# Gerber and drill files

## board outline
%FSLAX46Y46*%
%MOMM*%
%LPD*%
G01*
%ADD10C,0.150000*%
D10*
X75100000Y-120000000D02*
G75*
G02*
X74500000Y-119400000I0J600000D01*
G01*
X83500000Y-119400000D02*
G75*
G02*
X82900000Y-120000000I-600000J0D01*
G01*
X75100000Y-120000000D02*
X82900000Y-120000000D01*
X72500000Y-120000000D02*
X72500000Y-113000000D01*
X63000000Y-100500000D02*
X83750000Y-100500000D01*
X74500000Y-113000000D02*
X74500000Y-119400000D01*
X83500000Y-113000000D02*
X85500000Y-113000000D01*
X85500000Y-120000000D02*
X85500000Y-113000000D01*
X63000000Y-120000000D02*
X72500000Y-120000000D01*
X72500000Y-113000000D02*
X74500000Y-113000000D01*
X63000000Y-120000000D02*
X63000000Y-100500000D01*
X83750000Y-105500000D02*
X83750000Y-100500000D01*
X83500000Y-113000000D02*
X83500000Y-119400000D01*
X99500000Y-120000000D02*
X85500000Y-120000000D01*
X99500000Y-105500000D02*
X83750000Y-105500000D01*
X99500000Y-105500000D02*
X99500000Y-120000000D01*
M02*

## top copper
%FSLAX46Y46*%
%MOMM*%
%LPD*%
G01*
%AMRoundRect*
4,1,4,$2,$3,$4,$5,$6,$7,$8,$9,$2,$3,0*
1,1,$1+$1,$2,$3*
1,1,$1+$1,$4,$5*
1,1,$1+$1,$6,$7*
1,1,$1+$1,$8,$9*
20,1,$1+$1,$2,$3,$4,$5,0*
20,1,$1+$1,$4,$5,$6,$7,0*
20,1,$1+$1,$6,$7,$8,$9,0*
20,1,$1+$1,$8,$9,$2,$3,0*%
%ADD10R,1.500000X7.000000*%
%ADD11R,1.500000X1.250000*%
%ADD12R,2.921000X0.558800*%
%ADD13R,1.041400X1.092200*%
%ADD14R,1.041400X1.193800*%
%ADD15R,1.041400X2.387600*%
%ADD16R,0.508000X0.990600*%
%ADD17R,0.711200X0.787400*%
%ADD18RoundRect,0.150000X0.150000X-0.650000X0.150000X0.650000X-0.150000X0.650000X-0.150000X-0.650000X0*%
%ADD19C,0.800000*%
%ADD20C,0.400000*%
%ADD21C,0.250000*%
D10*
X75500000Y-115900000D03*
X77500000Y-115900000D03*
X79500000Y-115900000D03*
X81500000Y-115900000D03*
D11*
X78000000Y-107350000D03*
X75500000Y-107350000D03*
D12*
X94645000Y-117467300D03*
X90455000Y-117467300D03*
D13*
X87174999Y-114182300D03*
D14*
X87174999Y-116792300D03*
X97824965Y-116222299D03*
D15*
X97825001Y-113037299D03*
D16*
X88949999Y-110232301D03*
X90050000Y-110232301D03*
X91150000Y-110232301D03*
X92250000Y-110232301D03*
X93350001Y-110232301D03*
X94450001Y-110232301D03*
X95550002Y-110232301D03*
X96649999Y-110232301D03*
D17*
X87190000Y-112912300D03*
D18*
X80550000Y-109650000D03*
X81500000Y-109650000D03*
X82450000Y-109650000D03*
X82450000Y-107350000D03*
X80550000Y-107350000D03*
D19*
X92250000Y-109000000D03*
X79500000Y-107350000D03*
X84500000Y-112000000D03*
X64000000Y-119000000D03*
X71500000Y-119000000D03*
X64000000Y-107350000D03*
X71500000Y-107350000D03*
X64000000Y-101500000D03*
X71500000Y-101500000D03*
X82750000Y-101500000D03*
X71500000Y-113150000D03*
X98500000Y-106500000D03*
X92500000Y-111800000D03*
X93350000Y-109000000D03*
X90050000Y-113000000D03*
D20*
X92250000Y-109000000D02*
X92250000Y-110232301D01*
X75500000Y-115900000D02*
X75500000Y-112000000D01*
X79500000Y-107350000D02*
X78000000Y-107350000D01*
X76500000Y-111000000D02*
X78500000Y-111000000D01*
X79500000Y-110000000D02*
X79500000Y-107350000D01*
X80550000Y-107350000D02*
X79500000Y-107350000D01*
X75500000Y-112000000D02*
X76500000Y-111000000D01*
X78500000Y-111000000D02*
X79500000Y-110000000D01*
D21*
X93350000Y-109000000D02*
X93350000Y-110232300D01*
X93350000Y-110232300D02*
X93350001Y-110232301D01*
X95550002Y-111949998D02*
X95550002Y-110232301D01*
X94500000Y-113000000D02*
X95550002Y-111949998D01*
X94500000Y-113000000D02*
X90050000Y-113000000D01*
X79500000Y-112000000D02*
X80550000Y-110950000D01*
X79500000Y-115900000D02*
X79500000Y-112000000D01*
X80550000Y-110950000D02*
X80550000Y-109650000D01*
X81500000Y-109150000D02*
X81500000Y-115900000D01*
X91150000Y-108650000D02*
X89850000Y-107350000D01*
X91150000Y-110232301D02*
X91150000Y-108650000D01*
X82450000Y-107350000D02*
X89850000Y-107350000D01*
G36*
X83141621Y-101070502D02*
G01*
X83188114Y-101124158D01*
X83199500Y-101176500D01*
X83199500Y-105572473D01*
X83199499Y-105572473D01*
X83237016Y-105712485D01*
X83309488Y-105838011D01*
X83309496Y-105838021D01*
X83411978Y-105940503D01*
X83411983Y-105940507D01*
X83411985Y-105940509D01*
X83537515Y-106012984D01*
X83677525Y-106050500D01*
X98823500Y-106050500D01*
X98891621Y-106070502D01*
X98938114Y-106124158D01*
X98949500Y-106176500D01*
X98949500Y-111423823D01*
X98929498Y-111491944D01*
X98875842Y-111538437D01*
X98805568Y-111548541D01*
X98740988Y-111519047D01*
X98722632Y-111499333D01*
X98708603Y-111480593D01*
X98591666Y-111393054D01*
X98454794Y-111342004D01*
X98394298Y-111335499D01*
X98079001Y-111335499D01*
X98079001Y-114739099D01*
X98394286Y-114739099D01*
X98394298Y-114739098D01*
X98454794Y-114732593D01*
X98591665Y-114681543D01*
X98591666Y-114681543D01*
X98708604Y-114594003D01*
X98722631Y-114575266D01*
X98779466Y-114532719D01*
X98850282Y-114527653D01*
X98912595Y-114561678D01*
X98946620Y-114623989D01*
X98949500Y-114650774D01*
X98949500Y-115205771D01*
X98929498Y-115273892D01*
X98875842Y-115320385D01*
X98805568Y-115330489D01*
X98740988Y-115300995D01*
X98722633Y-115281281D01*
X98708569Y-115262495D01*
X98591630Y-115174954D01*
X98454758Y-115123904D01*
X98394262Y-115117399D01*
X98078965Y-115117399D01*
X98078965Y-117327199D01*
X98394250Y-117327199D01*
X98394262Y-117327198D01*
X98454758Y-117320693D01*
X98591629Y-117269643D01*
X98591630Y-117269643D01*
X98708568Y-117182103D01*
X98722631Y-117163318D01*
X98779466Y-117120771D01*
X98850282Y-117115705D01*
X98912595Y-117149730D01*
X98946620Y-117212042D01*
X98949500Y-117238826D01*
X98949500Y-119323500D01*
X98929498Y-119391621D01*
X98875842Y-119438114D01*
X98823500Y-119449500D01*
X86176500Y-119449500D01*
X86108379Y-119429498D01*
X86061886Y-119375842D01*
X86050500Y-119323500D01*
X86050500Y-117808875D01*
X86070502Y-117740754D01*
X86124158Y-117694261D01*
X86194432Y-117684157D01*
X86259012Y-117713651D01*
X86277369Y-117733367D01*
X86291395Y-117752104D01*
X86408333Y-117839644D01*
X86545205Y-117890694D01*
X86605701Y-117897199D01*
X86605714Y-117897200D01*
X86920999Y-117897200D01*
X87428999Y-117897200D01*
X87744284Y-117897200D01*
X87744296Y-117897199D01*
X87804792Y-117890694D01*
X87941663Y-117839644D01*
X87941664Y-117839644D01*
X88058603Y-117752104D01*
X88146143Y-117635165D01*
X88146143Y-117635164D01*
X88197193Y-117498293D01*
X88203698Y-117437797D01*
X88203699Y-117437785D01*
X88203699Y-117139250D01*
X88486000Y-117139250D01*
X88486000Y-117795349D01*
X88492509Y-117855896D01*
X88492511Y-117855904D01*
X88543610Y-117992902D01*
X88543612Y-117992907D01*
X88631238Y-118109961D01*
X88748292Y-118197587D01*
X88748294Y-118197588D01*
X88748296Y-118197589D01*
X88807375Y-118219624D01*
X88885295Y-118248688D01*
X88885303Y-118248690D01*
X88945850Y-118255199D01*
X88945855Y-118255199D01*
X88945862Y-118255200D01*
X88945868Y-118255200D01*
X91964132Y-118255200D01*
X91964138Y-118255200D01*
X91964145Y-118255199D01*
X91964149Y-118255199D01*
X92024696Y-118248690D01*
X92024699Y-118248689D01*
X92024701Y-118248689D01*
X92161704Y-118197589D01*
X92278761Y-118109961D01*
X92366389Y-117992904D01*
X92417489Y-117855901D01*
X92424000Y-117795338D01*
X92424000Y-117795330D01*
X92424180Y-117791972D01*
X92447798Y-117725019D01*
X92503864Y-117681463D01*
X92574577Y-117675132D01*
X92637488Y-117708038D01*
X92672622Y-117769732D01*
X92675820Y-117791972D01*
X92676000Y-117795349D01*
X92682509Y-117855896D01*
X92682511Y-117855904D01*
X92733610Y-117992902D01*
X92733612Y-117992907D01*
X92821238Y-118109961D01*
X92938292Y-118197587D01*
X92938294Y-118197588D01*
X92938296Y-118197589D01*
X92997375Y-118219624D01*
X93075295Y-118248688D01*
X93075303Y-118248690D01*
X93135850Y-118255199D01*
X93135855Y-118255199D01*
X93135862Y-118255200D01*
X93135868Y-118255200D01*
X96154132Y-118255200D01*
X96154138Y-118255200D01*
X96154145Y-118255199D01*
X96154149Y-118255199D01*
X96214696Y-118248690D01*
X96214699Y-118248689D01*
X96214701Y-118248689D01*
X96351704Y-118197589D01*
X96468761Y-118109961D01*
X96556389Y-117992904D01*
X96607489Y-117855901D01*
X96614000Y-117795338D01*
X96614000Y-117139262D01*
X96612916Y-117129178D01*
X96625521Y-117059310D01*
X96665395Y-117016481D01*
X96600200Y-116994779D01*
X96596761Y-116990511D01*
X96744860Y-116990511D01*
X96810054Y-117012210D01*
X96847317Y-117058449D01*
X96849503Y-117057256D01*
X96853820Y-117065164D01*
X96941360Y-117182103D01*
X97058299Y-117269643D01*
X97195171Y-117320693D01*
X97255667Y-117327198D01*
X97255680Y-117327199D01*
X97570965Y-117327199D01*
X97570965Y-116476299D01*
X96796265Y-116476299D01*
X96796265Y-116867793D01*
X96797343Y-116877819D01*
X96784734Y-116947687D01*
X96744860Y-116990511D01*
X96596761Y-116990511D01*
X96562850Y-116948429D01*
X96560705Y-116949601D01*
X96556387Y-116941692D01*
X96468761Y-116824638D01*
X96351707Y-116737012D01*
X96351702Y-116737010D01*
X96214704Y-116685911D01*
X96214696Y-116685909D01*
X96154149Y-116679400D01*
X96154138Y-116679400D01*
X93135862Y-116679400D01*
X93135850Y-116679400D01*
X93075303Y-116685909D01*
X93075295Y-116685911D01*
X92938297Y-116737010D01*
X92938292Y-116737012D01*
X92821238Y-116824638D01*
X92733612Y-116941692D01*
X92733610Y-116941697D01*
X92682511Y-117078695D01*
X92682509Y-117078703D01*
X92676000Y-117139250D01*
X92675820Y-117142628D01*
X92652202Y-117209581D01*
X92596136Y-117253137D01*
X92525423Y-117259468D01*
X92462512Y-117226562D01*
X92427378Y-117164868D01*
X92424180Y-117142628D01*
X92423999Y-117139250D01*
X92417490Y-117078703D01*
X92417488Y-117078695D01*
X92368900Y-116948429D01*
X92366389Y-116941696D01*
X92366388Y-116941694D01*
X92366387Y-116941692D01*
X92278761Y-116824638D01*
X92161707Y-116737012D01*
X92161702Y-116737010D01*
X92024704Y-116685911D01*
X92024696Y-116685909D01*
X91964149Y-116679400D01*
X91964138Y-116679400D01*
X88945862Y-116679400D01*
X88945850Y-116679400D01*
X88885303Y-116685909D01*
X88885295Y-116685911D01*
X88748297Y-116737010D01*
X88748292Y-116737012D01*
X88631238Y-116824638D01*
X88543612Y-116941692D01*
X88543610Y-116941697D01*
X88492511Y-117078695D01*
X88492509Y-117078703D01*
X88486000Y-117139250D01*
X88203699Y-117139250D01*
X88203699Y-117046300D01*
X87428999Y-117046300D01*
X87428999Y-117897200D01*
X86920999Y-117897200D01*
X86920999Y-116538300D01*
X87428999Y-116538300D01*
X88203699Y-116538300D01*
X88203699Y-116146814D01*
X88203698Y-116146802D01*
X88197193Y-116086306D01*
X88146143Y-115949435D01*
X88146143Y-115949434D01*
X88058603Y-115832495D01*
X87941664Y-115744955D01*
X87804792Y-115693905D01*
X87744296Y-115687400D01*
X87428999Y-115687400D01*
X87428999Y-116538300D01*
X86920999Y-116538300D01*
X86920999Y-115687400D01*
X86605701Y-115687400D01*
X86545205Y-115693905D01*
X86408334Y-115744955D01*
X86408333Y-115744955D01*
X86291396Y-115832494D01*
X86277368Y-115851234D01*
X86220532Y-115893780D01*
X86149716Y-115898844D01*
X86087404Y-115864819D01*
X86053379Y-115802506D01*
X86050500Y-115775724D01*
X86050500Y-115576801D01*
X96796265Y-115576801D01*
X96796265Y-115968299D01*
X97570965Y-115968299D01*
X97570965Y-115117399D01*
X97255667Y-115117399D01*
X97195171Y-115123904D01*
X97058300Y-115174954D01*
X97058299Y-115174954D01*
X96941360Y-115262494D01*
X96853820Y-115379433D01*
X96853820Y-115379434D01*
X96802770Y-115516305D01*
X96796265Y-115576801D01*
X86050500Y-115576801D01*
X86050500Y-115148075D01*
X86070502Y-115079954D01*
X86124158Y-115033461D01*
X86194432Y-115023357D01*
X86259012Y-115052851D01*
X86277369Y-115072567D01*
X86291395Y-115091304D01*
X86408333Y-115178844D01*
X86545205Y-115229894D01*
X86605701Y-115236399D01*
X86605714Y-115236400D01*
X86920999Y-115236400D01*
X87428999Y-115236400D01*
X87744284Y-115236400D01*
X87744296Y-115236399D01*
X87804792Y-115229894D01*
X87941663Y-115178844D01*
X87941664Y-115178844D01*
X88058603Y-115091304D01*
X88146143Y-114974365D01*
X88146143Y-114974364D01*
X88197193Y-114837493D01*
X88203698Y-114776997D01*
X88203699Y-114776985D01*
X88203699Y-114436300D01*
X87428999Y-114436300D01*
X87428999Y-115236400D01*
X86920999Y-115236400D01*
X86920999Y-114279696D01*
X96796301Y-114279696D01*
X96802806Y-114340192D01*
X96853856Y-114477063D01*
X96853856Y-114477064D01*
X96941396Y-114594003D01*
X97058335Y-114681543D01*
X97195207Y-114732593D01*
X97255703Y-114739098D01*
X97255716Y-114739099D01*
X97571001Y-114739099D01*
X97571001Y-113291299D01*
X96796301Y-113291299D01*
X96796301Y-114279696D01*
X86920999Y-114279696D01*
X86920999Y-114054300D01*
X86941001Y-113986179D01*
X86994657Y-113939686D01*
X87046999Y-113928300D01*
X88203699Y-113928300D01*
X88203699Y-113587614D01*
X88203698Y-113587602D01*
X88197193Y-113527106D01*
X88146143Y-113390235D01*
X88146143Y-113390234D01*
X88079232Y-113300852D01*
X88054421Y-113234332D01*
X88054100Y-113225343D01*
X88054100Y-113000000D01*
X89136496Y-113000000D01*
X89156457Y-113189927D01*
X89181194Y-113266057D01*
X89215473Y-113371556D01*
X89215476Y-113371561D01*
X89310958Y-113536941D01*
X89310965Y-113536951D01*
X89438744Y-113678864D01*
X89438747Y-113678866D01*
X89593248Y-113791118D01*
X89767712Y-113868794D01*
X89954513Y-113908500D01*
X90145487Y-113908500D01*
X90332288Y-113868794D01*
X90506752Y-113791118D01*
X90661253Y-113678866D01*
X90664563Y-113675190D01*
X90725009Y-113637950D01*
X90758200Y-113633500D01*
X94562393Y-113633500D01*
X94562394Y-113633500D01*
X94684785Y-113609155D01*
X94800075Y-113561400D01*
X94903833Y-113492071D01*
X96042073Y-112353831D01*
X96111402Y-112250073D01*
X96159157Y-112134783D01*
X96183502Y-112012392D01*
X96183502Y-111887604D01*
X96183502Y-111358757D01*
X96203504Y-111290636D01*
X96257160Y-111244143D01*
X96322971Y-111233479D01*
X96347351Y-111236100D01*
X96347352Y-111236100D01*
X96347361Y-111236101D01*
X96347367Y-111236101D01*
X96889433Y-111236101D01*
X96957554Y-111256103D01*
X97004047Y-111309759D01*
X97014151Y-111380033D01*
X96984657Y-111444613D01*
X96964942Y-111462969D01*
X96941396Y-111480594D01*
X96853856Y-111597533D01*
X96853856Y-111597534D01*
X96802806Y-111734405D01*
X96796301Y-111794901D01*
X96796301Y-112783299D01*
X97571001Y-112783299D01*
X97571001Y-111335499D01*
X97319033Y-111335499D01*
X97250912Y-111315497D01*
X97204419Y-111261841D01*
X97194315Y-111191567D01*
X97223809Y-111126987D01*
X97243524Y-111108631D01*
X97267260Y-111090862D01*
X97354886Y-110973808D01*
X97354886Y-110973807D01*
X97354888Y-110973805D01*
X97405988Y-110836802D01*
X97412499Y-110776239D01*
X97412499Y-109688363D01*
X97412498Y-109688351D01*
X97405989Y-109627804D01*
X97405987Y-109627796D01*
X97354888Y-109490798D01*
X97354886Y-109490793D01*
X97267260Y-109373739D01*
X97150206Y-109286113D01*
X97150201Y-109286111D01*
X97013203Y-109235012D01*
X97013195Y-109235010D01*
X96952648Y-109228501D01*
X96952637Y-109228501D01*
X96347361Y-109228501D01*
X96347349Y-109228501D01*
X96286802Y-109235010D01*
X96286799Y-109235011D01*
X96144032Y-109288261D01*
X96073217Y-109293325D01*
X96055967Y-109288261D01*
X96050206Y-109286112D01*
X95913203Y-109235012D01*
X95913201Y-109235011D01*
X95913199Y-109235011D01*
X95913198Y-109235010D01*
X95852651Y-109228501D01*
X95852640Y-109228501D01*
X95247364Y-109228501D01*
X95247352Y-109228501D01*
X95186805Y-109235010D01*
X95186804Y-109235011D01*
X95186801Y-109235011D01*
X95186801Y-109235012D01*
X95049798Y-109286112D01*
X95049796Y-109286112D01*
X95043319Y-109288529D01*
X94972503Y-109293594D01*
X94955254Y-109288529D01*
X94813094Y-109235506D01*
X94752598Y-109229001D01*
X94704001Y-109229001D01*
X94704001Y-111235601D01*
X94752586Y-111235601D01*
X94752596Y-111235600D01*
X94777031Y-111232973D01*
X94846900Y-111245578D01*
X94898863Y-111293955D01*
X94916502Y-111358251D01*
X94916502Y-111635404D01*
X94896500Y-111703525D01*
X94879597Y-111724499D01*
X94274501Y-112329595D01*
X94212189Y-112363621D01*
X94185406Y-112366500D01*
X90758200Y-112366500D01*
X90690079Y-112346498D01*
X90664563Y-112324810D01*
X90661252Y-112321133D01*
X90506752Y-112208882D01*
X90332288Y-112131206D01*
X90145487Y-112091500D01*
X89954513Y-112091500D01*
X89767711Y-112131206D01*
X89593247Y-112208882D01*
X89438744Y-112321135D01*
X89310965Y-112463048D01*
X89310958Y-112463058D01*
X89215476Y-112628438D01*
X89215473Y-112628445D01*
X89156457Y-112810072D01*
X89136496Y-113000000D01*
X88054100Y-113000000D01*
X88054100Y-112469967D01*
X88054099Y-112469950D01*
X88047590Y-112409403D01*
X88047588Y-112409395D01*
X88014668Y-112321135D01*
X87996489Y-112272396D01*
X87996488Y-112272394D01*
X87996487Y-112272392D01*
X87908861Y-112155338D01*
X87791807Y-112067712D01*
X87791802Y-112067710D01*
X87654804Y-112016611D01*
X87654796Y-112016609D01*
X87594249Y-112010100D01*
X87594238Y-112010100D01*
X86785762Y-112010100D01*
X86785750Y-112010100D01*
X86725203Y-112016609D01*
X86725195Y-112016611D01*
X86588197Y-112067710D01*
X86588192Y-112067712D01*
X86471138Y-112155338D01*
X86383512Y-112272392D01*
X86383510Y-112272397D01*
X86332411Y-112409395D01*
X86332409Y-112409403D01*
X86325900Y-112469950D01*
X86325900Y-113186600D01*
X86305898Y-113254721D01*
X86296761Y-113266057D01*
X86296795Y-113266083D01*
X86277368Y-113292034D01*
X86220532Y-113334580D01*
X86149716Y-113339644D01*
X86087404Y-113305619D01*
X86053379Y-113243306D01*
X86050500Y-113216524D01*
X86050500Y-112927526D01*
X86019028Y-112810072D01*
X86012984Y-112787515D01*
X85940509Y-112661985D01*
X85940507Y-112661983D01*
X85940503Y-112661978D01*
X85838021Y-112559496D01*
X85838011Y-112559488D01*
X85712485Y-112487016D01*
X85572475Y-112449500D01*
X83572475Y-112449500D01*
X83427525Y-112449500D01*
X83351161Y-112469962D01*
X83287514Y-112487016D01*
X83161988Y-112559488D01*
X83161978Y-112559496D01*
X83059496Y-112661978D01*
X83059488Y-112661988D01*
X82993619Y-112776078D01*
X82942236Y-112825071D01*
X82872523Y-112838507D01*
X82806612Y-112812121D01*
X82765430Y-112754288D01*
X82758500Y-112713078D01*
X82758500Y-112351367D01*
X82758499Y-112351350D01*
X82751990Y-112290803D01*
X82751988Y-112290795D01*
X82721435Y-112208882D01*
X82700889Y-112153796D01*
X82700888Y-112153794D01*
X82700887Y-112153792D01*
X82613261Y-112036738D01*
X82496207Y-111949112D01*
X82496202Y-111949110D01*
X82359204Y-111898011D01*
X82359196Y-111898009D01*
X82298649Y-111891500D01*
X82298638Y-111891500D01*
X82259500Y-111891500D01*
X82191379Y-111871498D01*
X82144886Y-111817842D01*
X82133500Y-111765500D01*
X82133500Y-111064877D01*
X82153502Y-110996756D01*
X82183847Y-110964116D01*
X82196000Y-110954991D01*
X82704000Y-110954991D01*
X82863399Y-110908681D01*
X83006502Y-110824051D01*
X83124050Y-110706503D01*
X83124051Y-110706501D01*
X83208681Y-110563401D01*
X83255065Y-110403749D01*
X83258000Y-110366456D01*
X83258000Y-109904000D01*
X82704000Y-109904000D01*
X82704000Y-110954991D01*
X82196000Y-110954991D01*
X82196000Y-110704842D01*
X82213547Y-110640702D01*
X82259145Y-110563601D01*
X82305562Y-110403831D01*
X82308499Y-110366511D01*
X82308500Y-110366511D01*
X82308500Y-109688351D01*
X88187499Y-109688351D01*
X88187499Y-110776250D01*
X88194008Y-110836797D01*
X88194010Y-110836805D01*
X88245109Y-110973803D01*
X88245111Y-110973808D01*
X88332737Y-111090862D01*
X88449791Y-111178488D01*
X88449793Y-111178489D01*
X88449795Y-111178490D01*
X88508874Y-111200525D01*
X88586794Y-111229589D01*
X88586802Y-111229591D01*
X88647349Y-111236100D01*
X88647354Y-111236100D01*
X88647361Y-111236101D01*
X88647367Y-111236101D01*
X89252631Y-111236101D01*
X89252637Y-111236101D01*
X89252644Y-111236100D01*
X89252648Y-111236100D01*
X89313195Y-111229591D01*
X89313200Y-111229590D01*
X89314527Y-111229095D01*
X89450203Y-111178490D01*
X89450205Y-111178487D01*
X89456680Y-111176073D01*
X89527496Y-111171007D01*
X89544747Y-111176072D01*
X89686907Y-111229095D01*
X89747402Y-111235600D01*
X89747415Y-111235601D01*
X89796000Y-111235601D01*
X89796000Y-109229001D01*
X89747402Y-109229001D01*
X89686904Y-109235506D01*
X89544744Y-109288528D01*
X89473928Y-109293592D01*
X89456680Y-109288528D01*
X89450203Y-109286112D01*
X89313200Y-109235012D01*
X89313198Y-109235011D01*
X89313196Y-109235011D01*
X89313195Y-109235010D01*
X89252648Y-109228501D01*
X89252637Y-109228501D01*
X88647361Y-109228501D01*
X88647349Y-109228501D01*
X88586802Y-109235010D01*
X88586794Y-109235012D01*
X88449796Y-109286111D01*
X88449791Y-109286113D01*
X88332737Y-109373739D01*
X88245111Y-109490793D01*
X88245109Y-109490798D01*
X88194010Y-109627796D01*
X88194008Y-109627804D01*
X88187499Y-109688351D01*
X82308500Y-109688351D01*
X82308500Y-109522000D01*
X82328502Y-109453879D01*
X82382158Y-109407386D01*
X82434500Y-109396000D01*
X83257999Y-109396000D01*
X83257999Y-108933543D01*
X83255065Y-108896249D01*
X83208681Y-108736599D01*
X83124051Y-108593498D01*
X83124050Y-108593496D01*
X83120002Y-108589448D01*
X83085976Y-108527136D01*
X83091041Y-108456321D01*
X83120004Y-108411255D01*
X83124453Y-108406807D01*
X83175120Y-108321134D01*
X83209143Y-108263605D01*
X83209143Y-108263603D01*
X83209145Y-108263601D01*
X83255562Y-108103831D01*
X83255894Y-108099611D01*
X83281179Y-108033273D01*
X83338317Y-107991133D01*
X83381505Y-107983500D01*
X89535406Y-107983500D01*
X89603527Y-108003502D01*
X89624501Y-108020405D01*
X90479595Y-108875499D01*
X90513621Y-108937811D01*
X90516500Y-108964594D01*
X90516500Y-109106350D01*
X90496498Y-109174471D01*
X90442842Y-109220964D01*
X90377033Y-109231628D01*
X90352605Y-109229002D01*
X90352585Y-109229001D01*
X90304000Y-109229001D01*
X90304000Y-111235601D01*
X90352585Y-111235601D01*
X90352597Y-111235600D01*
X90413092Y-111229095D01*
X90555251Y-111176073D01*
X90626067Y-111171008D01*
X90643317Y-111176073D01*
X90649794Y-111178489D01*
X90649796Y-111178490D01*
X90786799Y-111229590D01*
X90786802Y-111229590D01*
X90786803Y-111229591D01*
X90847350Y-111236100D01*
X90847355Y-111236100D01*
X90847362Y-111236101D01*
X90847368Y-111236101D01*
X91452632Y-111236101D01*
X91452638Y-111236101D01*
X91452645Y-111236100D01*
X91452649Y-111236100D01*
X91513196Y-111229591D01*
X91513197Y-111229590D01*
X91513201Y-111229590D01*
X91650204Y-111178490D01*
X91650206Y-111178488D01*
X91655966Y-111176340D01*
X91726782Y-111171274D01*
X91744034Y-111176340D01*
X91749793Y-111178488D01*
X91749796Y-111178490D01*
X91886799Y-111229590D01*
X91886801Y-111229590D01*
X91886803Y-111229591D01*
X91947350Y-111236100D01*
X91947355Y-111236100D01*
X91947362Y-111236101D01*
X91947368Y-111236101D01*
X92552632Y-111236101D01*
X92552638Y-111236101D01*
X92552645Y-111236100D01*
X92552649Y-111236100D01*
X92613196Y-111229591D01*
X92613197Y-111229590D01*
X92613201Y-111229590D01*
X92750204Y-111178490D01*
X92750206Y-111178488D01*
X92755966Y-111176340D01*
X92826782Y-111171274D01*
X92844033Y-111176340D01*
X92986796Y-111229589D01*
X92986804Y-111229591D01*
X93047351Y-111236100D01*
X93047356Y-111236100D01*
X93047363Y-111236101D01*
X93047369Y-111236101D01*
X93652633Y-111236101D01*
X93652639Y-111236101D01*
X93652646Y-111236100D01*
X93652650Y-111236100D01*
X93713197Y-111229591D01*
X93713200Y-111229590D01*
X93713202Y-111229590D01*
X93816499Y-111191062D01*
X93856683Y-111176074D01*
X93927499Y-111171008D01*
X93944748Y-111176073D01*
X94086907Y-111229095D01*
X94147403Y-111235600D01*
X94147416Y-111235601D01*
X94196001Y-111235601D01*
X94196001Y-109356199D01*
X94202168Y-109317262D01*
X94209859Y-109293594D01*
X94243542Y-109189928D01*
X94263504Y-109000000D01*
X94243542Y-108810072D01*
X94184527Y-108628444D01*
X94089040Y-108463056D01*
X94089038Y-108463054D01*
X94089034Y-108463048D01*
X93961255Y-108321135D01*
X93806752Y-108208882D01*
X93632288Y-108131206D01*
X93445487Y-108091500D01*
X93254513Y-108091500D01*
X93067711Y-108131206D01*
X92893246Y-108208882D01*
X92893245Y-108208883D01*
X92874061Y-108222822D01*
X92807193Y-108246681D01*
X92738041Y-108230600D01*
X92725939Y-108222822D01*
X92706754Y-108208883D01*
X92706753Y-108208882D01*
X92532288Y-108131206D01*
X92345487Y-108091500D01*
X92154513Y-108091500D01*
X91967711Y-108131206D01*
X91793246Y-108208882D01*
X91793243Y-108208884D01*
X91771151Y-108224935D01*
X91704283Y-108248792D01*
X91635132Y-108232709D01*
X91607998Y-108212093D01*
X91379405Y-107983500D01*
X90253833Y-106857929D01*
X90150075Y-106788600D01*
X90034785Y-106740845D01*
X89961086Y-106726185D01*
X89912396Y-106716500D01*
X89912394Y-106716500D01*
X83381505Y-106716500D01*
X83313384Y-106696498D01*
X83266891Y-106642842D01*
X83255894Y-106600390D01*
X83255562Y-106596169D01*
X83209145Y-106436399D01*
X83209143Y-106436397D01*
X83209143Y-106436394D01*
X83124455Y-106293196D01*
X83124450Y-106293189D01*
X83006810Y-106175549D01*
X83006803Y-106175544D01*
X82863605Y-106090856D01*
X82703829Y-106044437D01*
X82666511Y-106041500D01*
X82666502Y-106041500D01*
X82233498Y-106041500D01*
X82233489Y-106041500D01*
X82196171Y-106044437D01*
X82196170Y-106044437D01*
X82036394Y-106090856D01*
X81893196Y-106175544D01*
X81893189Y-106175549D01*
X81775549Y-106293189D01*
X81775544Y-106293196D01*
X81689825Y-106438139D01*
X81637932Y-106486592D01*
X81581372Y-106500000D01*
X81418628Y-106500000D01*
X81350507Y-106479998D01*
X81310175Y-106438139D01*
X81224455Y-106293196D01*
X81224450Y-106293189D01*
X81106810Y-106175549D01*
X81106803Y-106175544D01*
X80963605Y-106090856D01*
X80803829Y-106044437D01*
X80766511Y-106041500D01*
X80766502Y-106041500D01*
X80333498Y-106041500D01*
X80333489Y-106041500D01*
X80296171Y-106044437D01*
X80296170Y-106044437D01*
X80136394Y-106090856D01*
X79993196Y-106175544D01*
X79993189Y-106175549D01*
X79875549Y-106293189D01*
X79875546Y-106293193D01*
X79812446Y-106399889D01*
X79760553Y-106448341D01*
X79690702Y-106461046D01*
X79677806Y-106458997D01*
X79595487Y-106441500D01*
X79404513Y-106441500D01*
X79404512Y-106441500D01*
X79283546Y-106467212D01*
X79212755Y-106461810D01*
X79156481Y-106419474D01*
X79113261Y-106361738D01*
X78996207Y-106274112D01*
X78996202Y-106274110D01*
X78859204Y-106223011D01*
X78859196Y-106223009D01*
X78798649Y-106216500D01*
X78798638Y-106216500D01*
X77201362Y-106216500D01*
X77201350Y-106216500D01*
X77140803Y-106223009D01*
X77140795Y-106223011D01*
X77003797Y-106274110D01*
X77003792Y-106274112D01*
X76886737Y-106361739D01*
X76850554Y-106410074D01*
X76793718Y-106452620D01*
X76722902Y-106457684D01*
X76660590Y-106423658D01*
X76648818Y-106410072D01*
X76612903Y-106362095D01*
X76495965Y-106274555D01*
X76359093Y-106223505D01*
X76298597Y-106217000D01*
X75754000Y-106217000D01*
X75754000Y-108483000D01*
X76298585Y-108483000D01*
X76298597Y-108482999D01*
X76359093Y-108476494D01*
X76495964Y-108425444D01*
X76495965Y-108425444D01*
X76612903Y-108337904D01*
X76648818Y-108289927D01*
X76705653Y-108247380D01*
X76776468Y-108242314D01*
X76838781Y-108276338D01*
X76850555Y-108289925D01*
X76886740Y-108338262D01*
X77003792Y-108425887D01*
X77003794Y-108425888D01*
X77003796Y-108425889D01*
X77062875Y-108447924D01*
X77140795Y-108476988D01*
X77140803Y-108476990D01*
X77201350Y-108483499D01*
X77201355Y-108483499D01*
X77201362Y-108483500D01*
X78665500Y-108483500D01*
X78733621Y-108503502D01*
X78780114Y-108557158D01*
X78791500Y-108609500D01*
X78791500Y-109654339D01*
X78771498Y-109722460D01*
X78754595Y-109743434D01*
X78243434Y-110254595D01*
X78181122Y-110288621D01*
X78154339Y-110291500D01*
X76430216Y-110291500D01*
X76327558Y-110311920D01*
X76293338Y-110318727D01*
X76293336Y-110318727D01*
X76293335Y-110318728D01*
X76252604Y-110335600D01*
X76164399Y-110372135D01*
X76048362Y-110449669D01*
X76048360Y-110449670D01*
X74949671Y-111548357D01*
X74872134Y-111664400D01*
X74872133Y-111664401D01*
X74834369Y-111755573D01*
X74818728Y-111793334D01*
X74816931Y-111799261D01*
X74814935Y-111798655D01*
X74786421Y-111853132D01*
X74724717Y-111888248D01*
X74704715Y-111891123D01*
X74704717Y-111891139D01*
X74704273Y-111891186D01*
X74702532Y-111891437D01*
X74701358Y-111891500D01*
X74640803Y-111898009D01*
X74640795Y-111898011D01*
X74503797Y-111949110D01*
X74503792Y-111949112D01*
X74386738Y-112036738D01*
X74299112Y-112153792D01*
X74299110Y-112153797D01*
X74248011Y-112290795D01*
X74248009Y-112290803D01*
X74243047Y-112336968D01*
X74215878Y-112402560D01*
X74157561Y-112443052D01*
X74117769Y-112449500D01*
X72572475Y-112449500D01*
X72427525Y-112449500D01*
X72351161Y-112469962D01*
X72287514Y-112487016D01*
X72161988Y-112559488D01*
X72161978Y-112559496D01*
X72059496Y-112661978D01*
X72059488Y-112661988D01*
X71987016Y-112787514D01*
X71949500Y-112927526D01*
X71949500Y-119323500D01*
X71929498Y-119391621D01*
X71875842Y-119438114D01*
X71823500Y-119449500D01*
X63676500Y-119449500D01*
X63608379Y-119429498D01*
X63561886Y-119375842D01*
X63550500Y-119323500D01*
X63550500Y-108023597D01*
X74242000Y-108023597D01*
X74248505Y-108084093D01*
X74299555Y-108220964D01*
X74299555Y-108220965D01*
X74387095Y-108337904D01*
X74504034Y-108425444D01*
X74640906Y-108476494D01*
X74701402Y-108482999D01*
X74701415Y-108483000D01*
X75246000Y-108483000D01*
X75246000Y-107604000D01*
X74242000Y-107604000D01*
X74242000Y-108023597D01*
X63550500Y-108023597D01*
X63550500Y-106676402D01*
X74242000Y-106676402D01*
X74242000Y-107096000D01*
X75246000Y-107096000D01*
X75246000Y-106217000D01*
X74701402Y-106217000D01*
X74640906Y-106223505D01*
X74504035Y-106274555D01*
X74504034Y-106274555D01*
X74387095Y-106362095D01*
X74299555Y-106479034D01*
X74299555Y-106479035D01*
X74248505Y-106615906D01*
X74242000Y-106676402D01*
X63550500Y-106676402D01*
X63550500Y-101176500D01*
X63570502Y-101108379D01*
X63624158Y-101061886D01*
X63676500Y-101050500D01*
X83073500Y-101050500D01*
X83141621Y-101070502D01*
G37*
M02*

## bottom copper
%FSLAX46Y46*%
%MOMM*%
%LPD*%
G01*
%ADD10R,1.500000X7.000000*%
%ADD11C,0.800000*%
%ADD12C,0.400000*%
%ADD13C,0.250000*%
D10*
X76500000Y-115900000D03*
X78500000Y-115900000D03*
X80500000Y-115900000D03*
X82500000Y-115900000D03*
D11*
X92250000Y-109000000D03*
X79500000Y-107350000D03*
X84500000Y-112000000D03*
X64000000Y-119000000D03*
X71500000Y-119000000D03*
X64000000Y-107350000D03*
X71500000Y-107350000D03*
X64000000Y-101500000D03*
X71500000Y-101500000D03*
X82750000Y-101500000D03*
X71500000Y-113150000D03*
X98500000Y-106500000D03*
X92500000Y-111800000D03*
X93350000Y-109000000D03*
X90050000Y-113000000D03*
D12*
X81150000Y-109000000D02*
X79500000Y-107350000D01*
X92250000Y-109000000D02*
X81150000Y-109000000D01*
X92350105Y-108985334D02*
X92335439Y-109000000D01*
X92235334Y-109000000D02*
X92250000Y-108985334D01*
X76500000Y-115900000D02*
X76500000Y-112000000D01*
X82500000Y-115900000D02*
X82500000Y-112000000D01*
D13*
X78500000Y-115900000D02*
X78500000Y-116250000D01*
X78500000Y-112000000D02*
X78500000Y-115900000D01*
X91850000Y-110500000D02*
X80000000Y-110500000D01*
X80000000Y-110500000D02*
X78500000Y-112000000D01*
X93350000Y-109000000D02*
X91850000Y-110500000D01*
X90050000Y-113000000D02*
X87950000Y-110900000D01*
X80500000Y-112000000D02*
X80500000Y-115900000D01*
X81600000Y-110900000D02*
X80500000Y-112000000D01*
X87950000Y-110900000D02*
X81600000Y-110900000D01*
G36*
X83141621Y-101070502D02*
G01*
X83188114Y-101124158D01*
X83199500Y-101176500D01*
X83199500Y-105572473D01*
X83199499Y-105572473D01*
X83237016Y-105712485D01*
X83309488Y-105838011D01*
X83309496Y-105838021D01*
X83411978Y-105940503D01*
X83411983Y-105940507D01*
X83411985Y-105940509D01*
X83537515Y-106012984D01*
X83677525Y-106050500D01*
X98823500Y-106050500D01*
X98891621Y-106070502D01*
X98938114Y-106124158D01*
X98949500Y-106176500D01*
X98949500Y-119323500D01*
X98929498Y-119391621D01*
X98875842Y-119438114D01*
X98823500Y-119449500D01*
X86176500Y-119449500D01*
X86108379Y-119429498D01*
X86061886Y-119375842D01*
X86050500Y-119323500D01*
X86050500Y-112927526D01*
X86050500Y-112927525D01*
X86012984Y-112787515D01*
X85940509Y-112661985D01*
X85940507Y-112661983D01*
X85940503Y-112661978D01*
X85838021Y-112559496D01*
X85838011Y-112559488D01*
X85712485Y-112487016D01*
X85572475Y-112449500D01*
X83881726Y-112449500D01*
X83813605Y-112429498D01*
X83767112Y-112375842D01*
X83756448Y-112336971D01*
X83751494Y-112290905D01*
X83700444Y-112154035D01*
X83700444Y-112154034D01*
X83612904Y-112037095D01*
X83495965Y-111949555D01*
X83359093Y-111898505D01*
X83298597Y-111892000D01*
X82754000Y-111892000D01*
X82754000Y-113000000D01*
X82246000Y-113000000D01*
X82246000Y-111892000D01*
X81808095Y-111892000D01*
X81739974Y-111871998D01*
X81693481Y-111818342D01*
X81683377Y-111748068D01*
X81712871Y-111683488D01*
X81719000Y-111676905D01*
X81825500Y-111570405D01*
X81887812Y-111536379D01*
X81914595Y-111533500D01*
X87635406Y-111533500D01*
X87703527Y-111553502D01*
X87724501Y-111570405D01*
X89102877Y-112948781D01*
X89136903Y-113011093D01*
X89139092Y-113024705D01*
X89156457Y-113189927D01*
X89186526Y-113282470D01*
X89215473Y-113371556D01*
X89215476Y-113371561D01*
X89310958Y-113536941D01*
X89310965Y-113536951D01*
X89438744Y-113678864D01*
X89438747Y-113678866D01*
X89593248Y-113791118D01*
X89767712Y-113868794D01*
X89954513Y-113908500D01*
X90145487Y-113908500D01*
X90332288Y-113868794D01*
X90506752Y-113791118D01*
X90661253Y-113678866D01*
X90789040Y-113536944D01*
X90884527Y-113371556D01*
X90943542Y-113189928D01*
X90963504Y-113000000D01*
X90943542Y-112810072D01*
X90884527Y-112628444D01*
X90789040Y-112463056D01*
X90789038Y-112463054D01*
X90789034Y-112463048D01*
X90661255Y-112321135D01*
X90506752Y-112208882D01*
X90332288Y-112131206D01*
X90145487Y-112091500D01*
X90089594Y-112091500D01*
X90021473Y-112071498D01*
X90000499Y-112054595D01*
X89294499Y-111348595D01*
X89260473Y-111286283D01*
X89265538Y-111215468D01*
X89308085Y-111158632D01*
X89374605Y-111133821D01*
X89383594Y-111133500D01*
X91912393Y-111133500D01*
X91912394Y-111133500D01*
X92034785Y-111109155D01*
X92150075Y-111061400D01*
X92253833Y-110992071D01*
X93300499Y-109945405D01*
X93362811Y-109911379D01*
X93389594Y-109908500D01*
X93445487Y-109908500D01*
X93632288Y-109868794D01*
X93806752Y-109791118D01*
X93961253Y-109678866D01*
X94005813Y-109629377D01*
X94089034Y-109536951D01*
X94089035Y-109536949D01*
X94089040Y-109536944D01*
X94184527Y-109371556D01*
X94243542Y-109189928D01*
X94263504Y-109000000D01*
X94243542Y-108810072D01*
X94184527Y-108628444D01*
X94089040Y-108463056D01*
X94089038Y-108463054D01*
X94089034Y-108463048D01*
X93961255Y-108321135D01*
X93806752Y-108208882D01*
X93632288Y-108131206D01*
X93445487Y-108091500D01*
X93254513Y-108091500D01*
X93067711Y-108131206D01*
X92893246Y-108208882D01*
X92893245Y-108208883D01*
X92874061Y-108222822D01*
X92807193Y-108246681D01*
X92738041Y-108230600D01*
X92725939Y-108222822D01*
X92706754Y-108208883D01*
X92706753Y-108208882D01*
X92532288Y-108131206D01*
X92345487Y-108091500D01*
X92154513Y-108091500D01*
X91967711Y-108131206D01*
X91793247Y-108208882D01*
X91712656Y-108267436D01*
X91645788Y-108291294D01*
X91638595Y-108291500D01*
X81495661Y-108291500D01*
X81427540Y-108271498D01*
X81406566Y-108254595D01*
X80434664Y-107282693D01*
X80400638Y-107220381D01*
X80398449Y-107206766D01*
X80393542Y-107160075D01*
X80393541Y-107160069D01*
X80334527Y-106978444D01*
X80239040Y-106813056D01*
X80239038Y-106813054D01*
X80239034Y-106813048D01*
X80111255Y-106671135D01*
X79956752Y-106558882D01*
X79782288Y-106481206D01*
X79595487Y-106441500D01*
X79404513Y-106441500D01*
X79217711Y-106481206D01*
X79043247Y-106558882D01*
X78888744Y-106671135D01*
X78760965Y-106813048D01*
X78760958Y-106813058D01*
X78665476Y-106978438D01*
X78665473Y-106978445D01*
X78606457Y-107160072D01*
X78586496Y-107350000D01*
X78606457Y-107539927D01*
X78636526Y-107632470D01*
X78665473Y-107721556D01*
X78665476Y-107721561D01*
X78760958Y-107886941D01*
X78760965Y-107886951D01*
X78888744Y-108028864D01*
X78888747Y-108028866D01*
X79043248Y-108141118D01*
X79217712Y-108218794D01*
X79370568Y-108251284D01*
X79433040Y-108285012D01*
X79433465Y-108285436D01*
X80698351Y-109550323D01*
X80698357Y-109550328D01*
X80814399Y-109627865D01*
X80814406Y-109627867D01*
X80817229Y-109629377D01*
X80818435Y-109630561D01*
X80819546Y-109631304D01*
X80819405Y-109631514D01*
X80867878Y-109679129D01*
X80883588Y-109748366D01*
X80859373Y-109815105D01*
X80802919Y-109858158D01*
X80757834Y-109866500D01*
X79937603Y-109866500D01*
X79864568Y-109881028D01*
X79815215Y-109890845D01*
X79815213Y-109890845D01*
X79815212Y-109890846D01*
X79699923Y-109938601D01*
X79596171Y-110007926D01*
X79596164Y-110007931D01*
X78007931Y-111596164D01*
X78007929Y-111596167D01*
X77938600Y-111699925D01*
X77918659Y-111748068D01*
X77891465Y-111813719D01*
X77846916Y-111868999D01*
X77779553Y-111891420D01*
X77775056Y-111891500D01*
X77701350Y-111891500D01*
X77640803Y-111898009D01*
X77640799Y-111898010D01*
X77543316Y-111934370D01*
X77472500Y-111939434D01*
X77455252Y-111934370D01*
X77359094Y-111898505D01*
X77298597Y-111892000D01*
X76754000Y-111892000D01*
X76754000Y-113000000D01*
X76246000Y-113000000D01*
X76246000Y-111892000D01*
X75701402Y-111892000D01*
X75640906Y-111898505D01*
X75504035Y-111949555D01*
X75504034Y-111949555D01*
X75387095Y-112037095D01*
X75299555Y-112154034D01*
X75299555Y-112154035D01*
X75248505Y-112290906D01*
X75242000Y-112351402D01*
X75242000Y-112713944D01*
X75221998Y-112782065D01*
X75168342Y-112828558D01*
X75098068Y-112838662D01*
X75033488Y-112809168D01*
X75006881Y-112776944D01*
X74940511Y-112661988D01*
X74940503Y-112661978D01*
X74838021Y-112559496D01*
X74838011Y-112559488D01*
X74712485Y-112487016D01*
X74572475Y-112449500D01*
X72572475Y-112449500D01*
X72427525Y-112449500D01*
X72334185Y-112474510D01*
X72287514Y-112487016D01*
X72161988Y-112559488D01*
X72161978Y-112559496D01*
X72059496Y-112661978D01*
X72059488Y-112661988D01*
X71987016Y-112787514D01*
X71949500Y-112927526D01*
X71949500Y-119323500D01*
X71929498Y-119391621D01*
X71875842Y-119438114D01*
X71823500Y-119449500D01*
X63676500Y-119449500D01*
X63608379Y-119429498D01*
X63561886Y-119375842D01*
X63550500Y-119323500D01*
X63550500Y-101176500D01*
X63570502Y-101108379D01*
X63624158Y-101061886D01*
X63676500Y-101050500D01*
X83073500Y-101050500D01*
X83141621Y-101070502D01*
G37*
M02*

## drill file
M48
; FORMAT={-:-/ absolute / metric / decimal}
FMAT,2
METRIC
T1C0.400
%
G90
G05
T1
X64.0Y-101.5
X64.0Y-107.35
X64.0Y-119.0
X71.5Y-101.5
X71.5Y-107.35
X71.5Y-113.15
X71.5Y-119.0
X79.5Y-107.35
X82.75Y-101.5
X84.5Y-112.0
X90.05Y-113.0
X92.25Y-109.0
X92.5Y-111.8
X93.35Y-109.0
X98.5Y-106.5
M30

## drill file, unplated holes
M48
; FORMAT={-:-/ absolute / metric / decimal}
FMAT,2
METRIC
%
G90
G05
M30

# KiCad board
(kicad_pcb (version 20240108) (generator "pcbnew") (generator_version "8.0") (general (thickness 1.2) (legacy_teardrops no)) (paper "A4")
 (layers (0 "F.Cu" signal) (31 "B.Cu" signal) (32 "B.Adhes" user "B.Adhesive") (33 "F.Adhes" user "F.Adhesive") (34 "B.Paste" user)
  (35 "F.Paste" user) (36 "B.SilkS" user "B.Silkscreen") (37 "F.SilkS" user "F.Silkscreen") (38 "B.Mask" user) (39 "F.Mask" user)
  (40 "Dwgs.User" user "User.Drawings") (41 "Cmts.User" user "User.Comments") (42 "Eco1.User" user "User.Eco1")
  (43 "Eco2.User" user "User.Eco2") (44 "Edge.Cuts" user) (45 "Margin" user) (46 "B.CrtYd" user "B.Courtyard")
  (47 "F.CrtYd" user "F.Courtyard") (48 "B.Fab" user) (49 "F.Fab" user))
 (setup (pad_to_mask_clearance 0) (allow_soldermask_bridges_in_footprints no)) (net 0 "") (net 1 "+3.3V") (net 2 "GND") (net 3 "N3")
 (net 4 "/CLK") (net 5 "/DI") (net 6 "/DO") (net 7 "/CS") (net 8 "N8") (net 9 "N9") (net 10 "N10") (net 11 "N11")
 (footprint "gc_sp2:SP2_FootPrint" (layer "F.Cu") (at 75.5 115.9)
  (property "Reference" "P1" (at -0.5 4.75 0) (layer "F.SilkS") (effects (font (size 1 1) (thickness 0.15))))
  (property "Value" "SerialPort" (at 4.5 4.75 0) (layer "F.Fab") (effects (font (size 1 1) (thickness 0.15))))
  (pad "1" smd rect (at 0 0) (size 1.5 7) (layers "F.Cu" "F.Mask") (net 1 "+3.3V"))
  (pad "2" smd rect (at 1 0) (size 1.5 7) (layers "B.Cu" "B.Mask") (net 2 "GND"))
  (pad "3" smd rect (at 2 0) (size 1.5 7) (layers "F.Cu" "F.Mask") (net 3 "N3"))
  (pad "4" smd rect (at 3 0) (size 1.5 7) (layers "B.Cu" "B.Mask") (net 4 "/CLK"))
  (pad "5" smd rect (at 4 0) (size 1.5 7) (layers "F.Cu" "F.Mask") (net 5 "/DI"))
  (pad "6" smd rect (at 5 0) (size 1.5 7) (layers "B.Cu" "B.Mask") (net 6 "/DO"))
  (pad "7" smd rect (at 6 0) (size 1.5 7) (layers "F.Cu" "F.Mask") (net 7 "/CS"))
  (pad "8" smd rect (at 7 0) (size 1.5 7) (layers "B.Cu" "B.Mask") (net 2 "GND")))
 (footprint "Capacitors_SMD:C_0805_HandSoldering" (layer "F.Cu") (at 76.75 107.35 180)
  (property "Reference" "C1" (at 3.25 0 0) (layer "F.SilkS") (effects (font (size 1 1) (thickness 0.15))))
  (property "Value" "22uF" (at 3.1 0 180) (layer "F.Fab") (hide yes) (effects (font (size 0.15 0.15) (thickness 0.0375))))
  (pad "1" smd rect (at -1.25 0 180) (size 1.5 1.25) (layers "F.Cu" "F.Paste" "F.Mask") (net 1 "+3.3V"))
  (pad "2" smd rect (at 1.25 0 180) (size 1.5 1.25) (layers "F.Cu" "F.Paste" "F.Mask") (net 2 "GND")))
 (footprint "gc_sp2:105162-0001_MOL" (layer "F.Cu") (at 92.5 113.75 180)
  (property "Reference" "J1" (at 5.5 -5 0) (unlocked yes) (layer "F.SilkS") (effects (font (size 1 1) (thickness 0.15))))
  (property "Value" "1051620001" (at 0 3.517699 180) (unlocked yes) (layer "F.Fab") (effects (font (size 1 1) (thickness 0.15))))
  (pad "14" smd rect (at -2.145 -3.7173 180) (size 2.921 0.5588) (layers "F.Cu" "F.Paste" "F.Mask"))
  (pad "15" smd rect (at 2.045 -3.7173 180) (size 2.921 0.5588) (layers "F.Cu" "F.Paste" "F.Mask"))
  (pad "G1" smd rect (at 5.325001 -0.4323 180) (size 1.0414 1.0922) (layers "F.Cu" "F.Paste" "F.Mask") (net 2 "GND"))
  (pad "G2" smd rect (at 5.325001 -3.0423 180) (size 1.0414 1.1938) (layers "F.Cu" "F.Paste" "F.Mask") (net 2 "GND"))
  (pad "G3" smd rect (at -5.324965 -2.472299 180) (size 1.0414 1.1938) (layers "F.Cu" "F.Paste" "F.Mask") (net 2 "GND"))
  (pad "G4" smd rect (at -5.325001 0.712701 180) (size 1.0414 2.3876) (layers "F.Cu" "F.Paste" "F.Mask") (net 2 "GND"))
  (pad "P1" smd rect (at 3.550001 3.517699 180) (size 0.508 0.9906) (layers "F.Cu" "F.Paste" "F.Mask") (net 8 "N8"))
  (pad "P2" smd rect (at 2.45 3.517699 180) (size 0.508 0.9906) (layers "F.Cu" "F.Paste" "F.Mask") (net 2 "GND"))
  (pad "P3" smd rect (at 1.35 3.517699 180) (size 0.508 0.9906) (layers "F.Cu" "F.Paste" "F.Mask") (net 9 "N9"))
  (pad "P4" smd rect (at 0.25 3.517699 180) (size 0.508 0.9906) (layers "F.Cu" "F.Paste" "F.Mask") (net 1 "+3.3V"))
  (pad "P5" smd rect (at -0.850001 3.517699 180) (size 0.508 0.9906) (layers "F.Cu" "F.Paste" "F.Mask") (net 4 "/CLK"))
  (pad "P6" smd rect (at -1.950001 3.517699 180) (size 0.508 0.9906) (layers "F.Cu" "F.Paste" "F.Mask") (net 2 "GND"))
  (pad "P7" smd rect (at -3.050002 3.517699 180) (size 0.508 0.9906) (layers "F.Cu" "F.Paste" "F.Mask") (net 6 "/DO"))
  (pad "P8" smd rect (at -4.149999 3.517699 180) (size 0.508 0.9906) (layers "F.Cu" "F.Paste" "F.Mask") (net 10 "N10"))
  (pad "P9" smd rect (at 5.31 0.8377 180) (size 0.7112 0.7874) (layers "F.Cu" "F.Paste" "F.Mask") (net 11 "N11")))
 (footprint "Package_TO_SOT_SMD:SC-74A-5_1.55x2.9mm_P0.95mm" (layer "F.Cu") (at 81.5 108.5 90)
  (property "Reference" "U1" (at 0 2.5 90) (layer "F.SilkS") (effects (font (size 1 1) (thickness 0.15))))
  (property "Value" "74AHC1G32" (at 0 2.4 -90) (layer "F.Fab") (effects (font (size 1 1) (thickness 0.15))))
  (pad "1" smd roundrect (at -1.15 -0.95 90) (size 1.6 0.6) (layers "F.Cu" "F.Paste" "F.Mask") (roundrect_rratio 0.25) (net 5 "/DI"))
  (pad "2" smd roundrect (at -1.15 0 90) (size 1.6 0.6) (layers "F.Cu" "F.Paste" "F.Mask") (roundrect_rratio 0.25) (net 7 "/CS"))
  (pad "3" smd roundrect (at -1.15 0.95 90) (size 1.6 0.6) (layers "F.Cu" "F.Paste" "F.Mask") (roundrect_rratio 0.25) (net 2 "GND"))
  (pad "4" smd roundrect (at 1.15 0.95 90) (size 1.6 0.6) (layers "F.Cu" "F.Paste" "F.Mask") (roundrect_rratio 0.25) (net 9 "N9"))
  (pad "5" smd roundrect (at 1.15 -0.95 90) (size 1.6 0.6) (layers "F.Cu" "F.Paste" "F.Mask") (roundrect_rratio 0.25) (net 1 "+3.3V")))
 (gr_arc (start 75.1 120) (mid 74.675736 119.824264) (end 74.5 119.4) (stroke (width 0.15) (type solid)) (layer "Edge.Cuts"))
 (gr_arc (start 83.5 119.4) (mid 83.324264 119.824264) (end 82.9 120) (stroke (width 0.15) (type solid)) (layer "Edge.Cuts"))
 (gr_line (start 75.1 120) (end 82.9 120) (stroke (width 0.15) (type solid)) (layer "Edge.Cuts"))
 (gr_line (start 72.5 120) (end 72.5 113) (stroke (width 0.15) (type solid)) (layer "Edge.Cuts"))
 (gr_line (start 63 100.5) (end 83.75 100.5) (stroke (width 0.15) (type solid)) (layer "Edge.Cuts"))
 (gr_line (start 74.5 113) (end 74.5 119.4) (stroke (width 0.15) (type solid)) (layer "Edge.Cuts"))
 (gr_line (start 83.5 113) (end 85.5 113) (stroke (width 0.15) (type solid)) (layer "Edge.Cuts"))
 (gr_line (start 85.5 120) (end 85.5 113) (stroke (width 0.15) (type solid)) (layer "Edge.Cuts"))
 (gr_line (start 63 120) (end 72.5 120) (stroke (width 0.15) (type solid)) (layer "Edge.Cuts"))
 (gr_line (start 72.5 113) (end 74.5 113) (stroke (width 0.15) (type solid)) (layer "Edge.Cuts"))
 (gr_line (start 63 120) (end 63 100.5) (stroke (width 0.15) (type solid)) (layer "Edge.Cuts"))
 (gr_line (start 83.75 105.5) (end 83.75 100.5) (stroke (width 0.15) (type solid)) (layer "Edge.Cuts"))
 (gr_line (start 83.5 113) (end 83.5 119.4) (stroke (width 0.15) (type solid)) (layer "Edge.Cuts"))
 (gr_line (start 99.5 120) (end 85.5 120) (stroke (width 0.15) (type solid)) (layer "Edge.Cuts"))
 (gr_line (start 99.5 105.5) (end 83.75 105.5) (stroke (width 0.15) (type solid)) (layer "Edge.Cuts"))
 (gr_line (start 99.5 105.5) (end 99.5 120) (stroke (width 0.15) (type solid)) (layer "Edge.Cuts"))
 (segment (start 92.25 109) (end 92.25 110.232301) (width 0.4) (layer "F.Cu") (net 1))
 (segment (start 75.5 115.9) (end 75.5 112) (width 0.4) (layer "F.Cu") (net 1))
 (segment (start 79.5 107.35) (end 78 107.35) (width 0.4) (layer "F.Cu") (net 1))
 (segment (start 76.5 111) (end 78.5 111) (width 0.4) (layer "F.Cu") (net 1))
 (segment (start 79.5 110) (end 79.5 107.35) (width 0.4) (layer "F.Cu") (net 1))
 (segment (start 80.55 107.35) (end 79.5 107.35) (width 0.4) (layer "F.Cu") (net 1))
 (segment (start 75.5 112) (end 76.5 111) (width 0.4) (layer "F.Cu") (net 1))
 (segment (start 78.5 111) (end 79.5 110) (width 0.4) (layer "F.Cu") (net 1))
 (via (at 92.25 109) (size 0.8) (drill 0.4) (layers "F.Cu" "B.Cu") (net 1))
 (via (at 79.5 107.35) (size 0.8) (drill 0.4) (layers "F.Cu" "B.Cu") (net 1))
 (segment (start 92.350105 108.985334) (end 92.335439 109) (width 0.4) (layer "B.Cu") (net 1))
 (segment (start 81.15 109) (end 79.5 107.35) (width 0.4) (layer "B.Cu") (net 1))
 (segment (start 92.25 109) (end 81.15 109) (width 0.4) (layer "B.Cu") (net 1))
 (segment (start 92.235334 109) (end 92.25 108.985334) (width 0.4) (layer "B.Cu") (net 1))
 (via (at 84.5 112) (size 0.8) (drill 0.4) (layers "F.Cu" "B.Cu") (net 2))
 (via (at 64 119) (size 0.8) (drill 0.4) (layers "F.Cu" "B.Cu") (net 2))
 (via (at 71.5 119) (size 0.8) (drill 0.4) (layers "F.Cu" "B.Cu") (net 2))
 (via (at 64 107.35) (size 0.8) (drill 0.4) (layers "F.Cu" "B.Cu") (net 2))
 (via (at 71.5 107.35) (size 0.8) (drill 0.4) (layers "F.Cu" "B.Cu") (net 2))
 (via (at 64 101.5) (size 0.8) (drill 0.4) (layers "F.Cu" "B.Cu") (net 2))
 (via (at 71.5 101.5) (size 0.8) (drill 0.4) (layers "F.Cu" "B.Cu") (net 2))
 (via (at 82.75 101.5) (size 0.8) (drill 0.4) (layers "F.Cu" "B.Cu") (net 2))
 (via (at 71.5 113.15) (size 0.8) (drill 0.4) (layers "F.Cu" "B.Cu") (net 2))
 (via (at 98.5 106.5) (size 0.8) (drill 0.4) (layers "F.Cu" "B.Cu") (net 2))
 (via (at 92.5 111.8) (size 0.8) (drill 0.4) (layers "F.Cu" "B.Cu") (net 2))
 (segment (start 76.5 115.9) (end 76.5 112) (width 0.4) (layer "B.Cu") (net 2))
 (segment (start 82.5 115.9) (end 82.5 112) (width 0.4) (layer "B.Cu") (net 2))
 (segment (start 93.35 109) (end 93.35 110.2323) (width 0.25) (layer "F.Cu") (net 4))
 (segment (start 93.35 110.2323) (end 93.350001 110.232301) (width 0.25) (layer "F.Cu") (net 4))
 (via (at 93.35 109) (size 0.8) (drill 0.4) (layers "F.Cu" "B.Cu") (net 4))
 (segment (start 78.5 115.9) (end 78.5 116.25) (width 0.25) (layer "B.Cu") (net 4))
 (segment (start 78.5 112) (end 78.5 115.9) (width 0.25) (layer "B.Cu") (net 4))
 (segment (start 91.85 110.5) (end 80 110.5) (width 0.25) (layer "B.Cu") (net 4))
 (segment (start 80 110.5) (end 78.5 112) (width 0.25) (layer "B.Cu") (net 4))
 (segment (start 93.35 109) (end 91.85 110.5) (width 0.25) (layer "B.Cu") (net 4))
 (segment (start 95.550002 111.949998) (end 95.550002 110.232301) (width 0.25) (layer "F.Cu") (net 6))
 (segment (start 94.5 113) (end 95.550002 111.949998) (width 0.25) (layer "F.Cu") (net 6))
 (segment (start 94.5 113) (end 90.05 113) (width 0.25) (layer "F.Cu") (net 6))
 (via (at 90.05 113) (size 0.8) (drill 0.4) (layers "F.Cu" "B.Cu") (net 6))
 (segment (start 90.05 113) (end 87.95 110.9) (width 0.25) (layer "B.Cu") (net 6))
 (segment (start 80.5 112) (end 80.5 115.9) (width 0.25) (layer "B.Cu") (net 6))
 (segment (start 81.6 110.9) (end 80.5 112) (width 0.25) (layer "B.Cu") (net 6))
 (segment (start 87.95 110.9) (end 81.6 110.9) (width 0.25) (layer "B.Cu") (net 6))
 (segment (start 79.5 112) (end 80.55 110.95) (width 0.25) (layer "F.Cu") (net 5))
 (segment (start 79.5 115.9) (end 79.5 112) (width 0.25) (layer "F.Cu") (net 5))
 (segment (start 80.55 110.95) (end 80.55 109.65) (width 0.25) (layer "F.Cu") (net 5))
 (segment (start 81.5 109.15) (end 81.5 115.9) (width 0.25) (layer "F.Cu") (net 7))
 (segment (start 91.15 108.65) (end 89.85 107.35) (width 0.25) (layer "F.Cu") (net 9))
 (segment (start 91.15 110.232301) (end 91.15 108.65) (width 0.25) (layer "F.Cu") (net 9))
 (segment (start 82.45 107.35) (end 89.85 107.35) (width 0.25) (layer "F.Cu") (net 9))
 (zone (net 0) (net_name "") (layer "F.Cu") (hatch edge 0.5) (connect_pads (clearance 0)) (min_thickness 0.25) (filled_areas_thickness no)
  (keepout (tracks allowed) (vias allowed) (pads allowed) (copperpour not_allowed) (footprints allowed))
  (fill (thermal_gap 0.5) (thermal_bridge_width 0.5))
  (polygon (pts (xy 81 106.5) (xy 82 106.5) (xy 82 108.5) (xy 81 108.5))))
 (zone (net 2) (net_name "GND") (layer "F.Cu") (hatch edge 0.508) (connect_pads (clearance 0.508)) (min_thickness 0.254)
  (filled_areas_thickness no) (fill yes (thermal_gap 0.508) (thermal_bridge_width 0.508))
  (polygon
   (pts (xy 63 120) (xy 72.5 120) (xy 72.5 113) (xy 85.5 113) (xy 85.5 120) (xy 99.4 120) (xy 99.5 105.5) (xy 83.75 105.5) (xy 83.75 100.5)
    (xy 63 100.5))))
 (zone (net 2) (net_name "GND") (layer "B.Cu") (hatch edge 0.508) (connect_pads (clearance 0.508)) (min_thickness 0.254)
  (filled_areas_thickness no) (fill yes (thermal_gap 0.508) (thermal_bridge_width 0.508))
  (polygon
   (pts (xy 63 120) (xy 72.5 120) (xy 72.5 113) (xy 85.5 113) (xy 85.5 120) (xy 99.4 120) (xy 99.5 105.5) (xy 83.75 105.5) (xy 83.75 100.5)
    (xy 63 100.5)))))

